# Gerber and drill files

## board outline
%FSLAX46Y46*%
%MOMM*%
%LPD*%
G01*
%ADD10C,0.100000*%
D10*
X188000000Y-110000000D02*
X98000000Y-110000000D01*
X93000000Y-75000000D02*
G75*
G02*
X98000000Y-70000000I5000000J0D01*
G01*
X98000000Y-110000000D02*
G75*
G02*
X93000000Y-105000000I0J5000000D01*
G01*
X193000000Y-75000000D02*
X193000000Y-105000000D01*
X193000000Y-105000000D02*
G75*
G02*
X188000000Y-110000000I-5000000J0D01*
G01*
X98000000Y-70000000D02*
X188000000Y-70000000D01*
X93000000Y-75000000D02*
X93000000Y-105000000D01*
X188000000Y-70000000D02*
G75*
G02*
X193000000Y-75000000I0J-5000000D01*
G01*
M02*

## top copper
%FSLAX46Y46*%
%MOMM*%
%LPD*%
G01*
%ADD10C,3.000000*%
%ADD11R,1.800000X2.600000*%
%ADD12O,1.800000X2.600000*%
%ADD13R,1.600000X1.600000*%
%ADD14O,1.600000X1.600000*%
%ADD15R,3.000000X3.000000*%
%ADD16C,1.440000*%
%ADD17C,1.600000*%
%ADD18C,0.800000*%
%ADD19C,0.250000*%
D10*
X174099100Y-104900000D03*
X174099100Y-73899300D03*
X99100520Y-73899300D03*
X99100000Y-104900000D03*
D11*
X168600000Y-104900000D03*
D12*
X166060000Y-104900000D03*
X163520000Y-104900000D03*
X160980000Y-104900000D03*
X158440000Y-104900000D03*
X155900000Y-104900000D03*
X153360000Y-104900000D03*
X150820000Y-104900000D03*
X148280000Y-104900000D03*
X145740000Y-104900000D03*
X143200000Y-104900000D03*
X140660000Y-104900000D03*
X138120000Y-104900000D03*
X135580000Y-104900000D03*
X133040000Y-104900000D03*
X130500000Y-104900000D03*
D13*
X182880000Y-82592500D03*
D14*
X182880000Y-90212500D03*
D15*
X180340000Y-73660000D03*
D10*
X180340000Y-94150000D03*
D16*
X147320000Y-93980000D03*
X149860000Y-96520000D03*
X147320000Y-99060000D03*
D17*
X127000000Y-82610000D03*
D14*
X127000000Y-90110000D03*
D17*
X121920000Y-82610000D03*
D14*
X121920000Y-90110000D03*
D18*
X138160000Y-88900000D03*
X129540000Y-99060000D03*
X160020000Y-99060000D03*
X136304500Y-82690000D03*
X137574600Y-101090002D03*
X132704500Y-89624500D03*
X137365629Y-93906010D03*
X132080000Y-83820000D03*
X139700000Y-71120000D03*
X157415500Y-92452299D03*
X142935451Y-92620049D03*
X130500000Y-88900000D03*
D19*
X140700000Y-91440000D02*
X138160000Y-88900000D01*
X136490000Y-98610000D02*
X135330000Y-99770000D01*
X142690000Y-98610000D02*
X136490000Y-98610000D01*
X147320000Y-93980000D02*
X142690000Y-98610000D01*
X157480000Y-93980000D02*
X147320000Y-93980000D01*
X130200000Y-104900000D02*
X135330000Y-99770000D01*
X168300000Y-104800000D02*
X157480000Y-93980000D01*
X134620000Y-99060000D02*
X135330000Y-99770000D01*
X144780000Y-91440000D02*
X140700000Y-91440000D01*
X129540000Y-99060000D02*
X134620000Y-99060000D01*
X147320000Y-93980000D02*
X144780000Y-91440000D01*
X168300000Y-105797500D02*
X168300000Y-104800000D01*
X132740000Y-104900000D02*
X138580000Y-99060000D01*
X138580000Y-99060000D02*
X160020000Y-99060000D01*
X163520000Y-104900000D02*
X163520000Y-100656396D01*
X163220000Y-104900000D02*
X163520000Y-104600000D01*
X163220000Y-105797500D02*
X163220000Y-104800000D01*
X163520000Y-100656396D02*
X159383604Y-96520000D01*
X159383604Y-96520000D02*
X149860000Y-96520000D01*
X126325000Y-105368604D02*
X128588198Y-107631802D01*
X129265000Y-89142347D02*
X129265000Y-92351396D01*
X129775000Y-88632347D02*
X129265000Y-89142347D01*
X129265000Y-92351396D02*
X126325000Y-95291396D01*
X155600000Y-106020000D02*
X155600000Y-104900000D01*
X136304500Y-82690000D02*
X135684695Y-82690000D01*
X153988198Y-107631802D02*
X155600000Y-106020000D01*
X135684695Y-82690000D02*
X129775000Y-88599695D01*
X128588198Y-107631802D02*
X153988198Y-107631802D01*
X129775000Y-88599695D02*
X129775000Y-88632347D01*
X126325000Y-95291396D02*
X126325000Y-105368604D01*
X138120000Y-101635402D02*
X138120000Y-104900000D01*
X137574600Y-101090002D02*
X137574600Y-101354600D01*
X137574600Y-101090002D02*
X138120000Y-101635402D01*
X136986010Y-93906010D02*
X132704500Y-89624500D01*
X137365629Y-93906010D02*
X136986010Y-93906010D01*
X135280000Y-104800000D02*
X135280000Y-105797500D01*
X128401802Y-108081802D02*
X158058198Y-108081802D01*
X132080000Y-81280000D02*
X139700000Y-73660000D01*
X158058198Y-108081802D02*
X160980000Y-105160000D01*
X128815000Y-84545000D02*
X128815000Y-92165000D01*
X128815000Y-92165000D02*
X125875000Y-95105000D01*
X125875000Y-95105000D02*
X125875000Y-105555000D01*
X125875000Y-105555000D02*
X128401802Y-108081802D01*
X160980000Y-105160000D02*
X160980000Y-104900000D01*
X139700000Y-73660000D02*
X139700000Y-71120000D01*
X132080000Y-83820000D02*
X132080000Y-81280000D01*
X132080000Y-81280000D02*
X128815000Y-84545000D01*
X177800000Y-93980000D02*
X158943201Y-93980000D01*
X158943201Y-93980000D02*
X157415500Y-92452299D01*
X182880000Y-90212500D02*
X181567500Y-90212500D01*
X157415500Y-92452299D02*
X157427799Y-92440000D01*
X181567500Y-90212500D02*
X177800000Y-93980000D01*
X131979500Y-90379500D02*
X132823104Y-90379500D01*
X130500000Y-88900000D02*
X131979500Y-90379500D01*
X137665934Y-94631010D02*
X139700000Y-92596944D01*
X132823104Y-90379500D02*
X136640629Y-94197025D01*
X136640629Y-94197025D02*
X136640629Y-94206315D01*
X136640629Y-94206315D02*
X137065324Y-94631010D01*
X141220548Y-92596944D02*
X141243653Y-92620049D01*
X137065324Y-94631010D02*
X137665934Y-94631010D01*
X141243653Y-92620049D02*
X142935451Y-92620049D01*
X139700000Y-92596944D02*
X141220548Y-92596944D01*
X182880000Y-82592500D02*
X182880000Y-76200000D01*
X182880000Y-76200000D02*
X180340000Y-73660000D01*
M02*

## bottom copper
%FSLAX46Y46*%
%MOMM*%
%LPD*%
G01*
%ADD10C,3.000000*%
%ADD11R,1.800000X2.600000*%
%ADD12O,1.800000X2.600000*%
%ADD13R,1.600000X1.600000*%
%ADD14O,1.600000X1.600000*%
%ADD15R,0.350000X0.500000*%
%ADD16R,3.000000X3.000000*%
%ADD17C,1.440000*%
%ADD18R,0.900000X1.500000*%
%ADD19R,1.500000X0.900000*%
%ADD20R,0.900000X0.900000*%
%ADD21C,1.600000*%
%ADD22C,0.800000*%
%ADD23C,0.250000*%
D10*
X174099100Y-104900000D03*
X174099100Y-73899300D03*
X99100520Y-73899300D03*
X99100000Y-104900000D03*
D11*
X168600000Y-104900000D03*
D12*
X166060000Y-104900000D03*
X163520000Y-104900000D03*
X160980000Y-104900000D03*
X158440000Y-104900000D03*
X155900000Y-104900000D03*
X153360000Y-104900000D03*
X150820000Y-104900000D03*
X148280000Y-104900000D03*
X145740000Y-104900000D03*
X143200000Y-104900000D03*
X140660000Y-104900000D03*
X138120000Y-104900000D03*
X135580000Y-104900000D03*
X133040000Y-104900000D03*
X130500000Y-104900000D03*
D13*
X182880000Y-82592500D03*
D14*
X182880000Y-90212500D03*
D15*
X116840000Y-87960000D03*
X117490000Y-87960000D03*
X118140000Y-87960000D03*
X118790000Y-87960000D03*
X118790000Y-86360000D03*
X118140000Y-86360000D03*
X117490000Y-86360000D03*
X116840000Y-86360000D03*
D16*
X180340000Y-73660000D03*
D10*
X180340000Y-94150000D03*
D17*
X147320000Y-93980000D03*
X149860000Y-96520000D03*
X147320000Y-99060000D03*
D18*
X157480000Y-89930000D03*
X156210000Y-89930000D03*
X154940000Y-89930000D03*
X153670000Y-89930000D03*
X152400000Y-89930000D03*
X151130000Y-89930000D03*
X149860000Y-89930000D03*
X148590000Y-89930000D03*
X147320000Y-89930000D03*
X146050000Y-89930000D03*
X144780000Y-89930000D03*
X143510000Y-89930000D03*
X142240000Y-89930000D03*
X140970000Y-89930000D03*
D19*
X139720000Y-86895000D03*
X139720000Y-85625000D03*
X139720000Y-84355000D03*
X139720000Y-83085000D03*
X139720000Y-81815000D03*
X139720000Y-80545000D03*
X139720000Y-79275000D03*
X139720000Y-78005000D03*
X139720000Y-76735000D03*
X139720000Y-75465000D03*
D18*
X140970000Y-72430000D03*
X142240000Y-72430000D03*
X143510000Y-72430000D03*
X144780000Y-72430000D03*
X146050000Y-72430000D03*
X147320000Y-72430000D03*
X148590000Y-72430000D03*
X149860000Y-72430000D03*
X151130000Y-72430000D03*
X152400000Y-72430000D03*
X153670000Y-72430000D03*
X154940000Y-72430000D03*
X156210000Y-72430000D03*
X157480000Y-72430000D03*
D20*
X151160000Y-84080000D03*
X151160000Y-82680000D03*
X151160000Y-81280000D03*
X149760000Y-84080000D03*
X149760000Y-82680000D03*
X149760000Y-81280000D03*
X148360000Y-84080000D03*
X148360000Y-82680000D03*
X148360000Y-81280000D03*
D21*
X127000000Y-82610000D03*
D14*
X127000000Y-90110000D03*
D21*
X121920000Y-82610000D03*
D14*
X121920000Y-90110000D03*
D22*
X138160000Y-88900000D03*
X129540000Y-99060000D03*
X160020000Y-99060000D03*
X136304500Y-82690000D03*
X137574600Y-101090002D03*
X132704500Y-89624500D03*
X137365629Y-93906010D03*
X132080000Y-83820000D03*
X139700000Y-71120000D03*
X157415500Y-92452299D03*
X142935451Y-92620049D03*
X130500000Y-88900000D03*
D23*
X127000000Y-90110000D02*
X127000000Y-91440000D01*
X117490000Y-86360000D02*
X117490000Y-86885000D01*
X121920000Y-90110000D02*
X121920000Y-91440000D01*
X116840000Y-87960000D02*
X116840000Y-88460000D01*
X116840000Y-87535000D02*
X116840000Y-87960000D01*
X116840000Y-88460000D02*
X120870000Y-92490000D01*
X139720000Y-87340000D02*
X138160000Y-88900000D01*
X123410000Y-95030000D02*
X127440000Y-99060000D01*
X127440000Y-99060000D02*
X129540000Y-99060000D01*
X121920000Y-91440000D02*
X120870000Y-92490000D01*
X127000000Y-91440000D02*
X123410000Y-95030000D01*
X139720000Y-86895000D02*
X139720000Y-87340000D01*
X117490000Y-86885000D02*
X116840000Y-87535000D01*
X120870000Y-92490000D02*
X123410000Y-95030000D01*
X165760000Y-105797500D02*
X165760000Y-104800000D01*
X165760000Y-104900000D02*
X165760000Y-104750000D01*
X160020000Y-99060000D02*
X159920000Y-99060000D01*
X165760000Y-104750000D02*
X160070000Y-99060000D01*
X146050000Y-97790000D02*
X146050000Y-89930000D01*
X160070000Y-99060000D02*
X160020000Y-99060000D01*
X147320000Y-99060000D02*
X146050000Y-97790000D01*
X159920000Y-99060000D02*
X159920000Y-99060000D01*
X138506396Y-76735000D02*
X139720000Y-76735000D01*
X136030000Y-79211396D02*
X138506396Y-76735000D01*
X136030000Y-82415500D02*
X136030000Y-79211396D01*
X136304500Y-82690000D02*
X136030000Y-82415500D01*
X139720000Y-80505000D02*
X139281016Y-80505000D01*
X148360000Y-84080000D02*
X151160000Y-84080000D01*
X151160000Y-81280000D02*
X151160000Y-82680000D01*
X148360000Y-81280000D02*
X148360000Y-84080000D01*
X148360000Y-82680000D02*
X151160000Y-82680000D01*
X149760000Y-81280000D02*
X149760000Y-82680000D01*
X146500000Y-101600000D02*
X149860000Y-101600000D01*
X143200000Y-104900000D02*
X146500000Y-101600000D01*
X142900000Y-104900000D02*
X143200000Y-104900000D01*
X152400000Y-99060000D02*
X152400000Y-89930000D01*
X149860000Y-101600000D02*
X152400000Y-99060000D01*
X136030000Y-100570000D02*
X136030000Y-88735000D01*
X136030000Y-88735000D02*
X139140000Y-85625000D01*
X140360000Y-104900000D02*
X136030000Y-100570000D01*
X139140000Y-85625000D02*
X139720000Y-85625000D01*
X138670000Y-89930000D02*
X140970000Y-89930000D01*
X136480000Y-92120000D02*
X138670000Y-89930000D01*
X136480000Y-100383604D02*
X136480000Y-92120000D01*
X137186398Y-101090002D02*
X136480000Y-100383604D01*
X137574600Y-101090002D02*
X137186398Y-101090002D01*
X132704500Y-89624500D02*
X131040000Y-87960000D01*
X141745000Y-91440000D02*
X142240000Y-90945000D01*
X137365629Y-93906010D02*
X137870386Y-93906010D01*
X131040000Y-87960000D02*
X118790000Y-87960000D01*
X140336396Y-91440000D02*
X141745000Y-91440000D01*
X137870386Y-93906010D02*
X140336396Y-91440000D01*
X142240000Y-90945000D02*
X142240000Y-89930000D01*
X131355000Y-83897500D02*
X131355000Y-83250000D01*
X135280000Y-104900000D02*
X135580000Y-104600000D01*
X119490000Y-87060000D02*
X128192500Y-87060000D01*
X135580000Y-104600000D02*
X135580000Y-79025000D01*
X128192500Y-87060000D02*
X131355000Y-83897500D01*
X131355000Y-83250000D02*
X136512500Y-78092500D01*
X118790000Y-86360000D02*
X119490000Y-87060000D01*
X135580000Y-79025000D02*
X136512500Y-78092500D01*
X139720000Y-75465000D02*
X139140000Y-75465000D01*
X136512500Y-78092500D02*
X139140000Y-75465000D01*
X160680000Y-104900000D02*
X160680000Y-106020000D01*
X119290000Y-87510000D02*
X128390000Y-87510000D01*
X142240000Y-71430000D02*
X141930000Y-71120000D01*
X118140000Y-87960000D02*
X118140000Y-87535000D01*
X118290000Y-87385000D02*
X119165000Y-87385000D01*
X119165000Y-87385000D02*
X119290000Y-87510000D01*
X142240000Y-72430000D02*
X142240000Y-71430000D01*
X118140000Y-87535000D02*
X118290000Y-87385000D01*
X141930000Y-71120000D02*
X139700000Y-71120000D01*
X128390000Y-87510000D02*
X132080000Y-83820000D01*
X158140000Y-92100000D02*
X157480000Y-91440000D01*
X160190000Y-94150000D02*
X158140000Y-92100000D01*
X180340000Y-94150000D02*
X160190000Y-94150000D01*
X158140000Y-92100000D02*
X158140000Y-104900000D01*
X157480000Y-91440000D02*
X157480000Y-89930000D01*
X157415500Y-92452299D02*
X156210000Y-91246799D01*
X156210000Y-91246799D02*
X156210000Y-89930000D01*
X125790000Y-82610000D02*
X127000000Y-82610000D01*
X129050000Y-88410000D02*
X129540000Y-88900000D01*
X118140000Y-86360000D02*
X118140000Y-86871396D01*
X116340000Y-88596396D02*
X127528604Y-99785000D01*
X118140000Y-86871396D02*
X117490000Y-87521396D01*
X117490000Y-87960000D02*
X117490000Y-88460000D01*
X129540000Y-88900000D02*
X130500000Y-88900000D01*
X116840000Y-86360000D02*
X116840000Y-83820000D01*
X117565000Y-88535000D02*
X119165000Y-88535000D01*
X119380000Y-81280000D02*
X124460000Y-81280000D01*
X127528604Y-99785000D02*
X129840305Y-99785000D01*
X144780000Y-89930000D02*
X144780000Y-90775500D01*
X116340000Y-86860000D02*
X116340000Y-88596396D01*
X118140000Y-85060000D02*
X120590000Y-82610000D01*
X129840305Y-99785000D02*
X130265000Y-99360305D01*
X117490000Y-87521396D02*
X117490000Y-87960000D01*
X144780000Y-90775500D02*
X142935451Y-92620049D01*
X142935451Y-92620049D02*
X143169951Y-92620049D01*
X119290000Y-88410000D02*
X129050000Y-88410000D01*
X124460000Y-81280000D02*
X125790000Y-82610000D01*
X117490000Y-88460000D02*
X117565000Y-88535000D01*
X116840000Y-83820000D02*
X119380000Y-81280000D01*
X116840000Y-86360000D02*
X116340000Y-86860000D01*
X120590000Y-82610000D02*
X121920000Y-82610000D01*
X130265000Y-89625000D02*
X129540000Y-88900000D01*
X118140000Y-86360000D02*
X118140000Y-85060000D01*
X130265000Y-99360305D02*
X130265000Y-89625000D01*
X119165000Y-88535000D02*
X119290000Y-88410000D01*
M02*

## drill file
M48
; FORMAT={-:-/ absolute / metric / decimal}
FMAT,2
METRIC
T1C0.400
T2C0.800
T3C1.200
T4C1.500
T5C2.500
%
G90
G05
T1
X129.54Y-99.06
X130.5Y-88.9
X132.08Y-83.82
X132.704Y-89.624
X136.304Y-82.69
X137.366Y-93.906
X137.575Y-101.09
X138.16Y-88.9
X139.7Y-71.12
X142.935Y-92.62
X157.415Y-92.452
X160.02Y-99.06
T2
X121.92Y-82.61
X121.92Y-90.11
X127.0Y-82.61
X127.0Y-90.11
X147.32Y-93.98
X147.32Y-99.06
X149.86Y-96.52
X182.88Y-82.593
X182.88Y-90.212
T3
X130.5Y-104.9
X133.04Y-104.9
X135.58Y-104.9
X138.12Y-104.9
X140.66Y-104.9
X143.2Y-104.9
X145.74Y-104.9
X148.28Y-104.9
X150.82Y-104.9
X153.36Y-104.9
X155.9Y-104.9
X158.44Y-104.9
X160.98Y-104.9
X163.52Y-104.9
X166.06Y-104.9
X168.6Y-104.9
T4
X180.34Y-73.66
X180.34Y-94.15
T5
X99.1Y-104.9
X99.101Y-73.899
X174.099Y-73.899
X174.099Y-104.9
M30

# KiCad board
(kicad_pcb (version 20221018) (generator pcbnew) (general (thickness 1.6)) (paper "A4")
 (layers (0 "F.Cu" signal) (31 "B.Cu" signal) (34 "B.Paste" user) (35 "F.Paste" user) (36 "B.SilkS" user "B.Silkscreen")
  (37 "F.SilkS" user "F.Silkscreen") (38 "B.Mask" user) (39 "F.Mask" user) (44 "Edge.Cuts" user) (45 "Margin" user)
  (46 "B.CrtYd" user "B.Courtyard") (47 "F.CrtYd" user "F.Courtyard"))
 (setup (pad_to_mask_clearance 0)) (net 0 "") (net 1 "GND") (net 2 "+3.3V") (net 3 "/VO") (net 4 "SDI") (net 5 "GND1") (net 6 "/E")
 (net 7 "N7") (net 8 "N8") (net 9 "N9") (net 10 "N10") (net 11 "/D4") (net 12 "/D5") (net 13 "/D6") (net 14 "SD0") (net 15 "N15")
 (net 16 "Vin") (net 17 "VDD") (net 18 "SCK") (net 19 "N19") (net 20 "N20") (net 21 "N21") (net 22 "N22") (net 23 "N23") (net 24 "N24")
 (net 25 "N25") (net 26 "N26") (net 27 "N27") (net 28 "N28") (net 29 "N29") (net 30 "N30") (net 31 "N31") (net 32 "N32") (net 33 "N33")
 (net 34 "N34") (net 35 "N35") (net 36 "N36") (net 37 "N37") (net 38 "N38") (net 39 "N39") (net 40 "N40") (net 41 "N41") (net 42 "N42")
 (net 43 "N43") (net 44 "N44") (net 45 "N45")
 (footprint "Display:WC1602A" (layer "F.Cu") (at 168.6 104.9 180)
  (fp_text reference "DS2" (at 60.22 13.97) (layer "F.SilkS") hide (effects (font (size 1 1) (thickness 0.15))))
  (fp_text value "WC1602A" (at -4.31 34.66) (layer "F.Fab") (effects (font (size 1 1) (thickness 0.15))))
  (pad "" thru_hole circle (at -5.4991 0 180) (size 3 3) (drill 2.5) (layers "*.Cu" "*.Mask"))
  (pad "" thru_hole circle (at -5.4991 31.0007 180) (size 3 3) (drill 2.5) (layers "*.Cu" "*.Mask"))
  (pad "" thru_hole circle (at 69.49948 31.0007 180) (size 3 3) (drill 2.5) (layers "*.Cu" "*.Mask"))
  (pad "" thru_hole circle (at 69.5 0 180) (size 3 3) (drill 2.5) (layers "*.Cu" "*.Mask"))
  (pad "1" thru_hole rect (at 0 0 180) (size 1.8 2.6) (drill 1.2) (layers "*.Cu" "*.Mask") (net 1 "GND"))
  (pad "2" thru_hole oval (at 2.54 0 180) (size 1.8 2.6) (drill 1.2) (layers "*.Cu" "*.Mask") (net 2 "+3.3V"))
  (pad "3" thru_hole oval (at 5.08 0 180) (size 1.8 2.6) (drill 1.2) (layers "*.Cu" "*.Mask") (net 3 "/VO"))
  (pad "4" thru_hole oval (at 7.62 0 180) (size 1.8 2.6) (drill 1.2) (layers "*.Cu" "*.Mask") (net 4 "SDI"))
  (pad "5" thru_hole oval (at 10.16 0 180) (size 1.8 2.6) (drill 1.2) (layers "*.Cu" "*.Mask") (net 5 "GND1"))
  (pad "6" thru_hole oval (at 12.7 0 180) (size 1.8 2.6) (drill 1.2) (layers "*.Cu" "*.Mask") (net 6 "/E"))
  (pad "7" thru_hole oval (at 15.24 0 180) (size 1.8 2.6) (drill 1.2) (layers "*.Cu" "*.Mask") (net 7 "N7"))
  (pad "8" thru_hole oval (at 17.78 0 180) (size 1.8 2.6) (drill 1.2) (layers "*.Cu" "*.Mask") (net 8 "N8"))
  (pad "9" thru_hole oval (at 20.32 0 180) (size 1.8 2.6) (drill 1.2) (layers "*.Cu" "*.Mask") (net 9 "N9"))
  (pad "10" thru_hole oval (at 22.86 0 180) (size 1.8 2.6) (drill 1.2) (layers "*.Cu" "*.Mask") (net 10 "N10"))
  (pad "11" thru_hole oval (at 25.4 0 180) (size 1.8 2.6) (drill 1.2) (layers "*.Cu" "*.Mask") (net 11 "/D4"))
  (pad "12" thru_hole oval (at 27.94 0 180) (size 1.8 2.6) (drill 1.2) (layers "*.Cu" "*.Mask") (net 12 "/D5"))
  (pad "13" thru_hole oval (at 30.48 0 180) (size 1.8 2.6) (drill 1.2) (layers "*.Cu" "*.Mask") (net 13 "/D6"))
  (pad "14" thru_hole oval (at 33.02 0 180) (size 1.8 2.6) (drill 1.2) (layers "*.Cu" "*.Mask") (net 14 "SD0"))
  (pad "15" thru_hole oval (at 35.56 0 180) (size 1.8 2.6) (drill 1.2) (layers "*.Cu" "*.Mask") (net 2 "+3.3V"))
  (pad "16" thru_hole oval (at 38.1 0 180) (size 1.8 2.6) (drill 1.2) (layers "*.Cu" "*.Mask") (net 1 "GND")))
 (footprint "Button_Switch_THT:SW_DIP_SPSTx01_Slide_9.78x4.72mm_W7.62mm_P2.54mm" (layer "F.Cu") (at 182.88 82.5925 -90)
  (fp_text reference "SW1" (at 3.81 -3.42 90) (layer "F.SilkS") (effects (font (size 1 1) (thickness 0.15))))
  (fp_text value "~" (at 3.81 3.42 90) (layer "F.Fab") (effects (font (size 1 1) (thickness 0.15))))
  (pad "1" thru_hole rect (at 0 0 270) (size 1.6 1.6) (drill 0.8) (layers "*.Cu" "*.Mask") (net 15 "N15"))
  (pad "2" thru_hole oval (at 7.62 0 270) (size 1.6 1.6) (drill 0.8) (layers "*.Cu" "*.Mask") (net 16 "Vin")))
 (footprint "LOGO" (layer "F.Cu") (at 185.42 101.6)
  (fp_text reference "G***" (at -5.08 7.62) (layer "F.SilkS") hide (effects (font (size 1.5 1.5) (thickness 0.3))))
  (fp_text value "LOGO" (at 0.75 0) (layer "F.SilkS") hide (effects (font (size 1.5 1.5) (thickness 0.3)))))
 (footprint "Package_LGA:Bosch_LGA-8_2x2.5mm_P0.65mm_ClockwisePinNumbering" (layer "B.Cu") (at 117.815 87.16)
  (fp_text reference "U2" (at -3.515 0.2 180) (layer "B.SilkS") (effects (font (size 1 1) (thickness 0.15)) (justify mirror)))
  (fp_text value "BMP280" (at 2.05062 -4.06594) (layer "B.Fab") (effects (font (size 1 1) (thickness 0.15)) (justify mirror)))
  (pad "1" smd rect (at -0.975 0.8 270) (size 0.5 0.35) (layers "B.Cu" "B.Paste" "B.Mask") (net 1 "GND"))
  (pad "2" smd rect (at -0.325 0.8 270) (size 0.5 0.35) (layers "B.Cu" "B.Paste" "B.Mask") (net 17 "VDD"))
  (pad "3" smd rect (at 0.325 0.8 270) (size 0.5 0.35) (layers "B.Cu" "B.Paste" "B.Mask") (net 4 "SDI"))
  (pad "4" smd rect (at 0.975 0.8 270) (size 0.5 0.35) (layers "B.Cu" "B.Paste" "B.Mask") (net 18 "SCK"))
  (pad "5" smd rect (at 0.975 -0.8 270) (size 0.5 0.35) (layers "B.Cu" "B.Paste" "B.Mask") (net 14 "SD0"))
  (pad "6" smd rect (at 0.325 -0.8 270) (size 0.5 0.35) (layers "B.Cu" "B.Paste" "B.Mask") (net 17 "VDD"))
  (pad "7" smd rect (at -0.325 -0.8 270) (size 0.5 0.35) (layers "B.Cu" "B.Paste" "B.Mask") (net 1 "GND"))
  (pad "8" smd rect (at -0.975 -0.8 270) (size 0.5 0.35) (layers "B.Cu" "B.Paste" "B.Mask") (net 17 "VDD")))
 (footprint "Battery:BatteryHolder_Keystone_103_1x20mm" (layer "B.Cu") (at 180.34 73.66 -90)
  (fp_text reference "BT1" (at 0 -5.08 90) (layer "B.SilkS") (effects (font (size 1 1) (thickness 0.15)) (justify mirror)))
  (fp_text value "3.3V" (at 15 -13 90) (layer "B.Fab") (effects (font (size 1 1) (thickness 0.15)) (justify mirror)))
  (pad "1" thru_hole rect (at 0 0 270) (size 3 3) (drill 1.5) (layers "*.Cu" "*.Mask") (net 15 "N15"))
  (pad "2" thru_hole circle (at 20.49 0 270) (size 3 3) (drill 1.5) (layers "*.Cu" "*.Mask") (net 5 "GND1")))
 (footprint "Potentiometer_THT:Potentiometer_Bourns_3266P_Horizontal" (layer "B.Cu") (at 147.32 93.98 180)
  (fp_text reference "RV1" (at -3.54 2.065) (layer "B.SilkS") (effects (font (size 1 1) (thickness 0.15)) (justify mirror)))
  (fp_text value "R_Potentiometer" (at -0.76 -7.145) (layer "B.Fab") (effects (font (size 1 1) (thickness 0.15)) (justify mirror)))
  (pad "1" thru_hole circle (at 0 0 180) (size 1.44 1.44) (drill 0.8) (layers "*.Cu" "*.Mask") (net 1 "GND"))
  (pad "2" thru_hole circle (at -2.54 -2.54 180) (size 1.44 1.44) (drill 0.8) (layers "*.Cu" "*.Mask") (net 3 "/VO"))
  (pad "3" thru_hole circle (at 0 -5.08 180) (size 1.44 1.44) (drill 0.8) (layers "*.Cu" "*.Mask") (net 2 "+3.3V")))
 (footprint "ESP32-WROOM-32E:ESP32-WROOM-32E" (layer "B.Cu") (at 149.225 81.18 90)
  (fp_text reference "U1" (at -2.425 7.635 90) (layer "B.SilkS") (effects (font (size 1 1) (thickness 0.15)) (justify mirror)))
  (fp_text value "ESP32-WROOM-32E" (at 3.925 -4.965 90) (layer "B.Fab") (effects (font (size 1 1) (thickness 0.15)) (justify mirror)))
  (pad "1" smd rect (at -8.75 8.255 90) (size 1.5 0.9) (layers "B.Cu" "B.Paste" "B.Mask") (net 5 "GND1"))
  (pad "2" smd rect (at -8.75 6.985 90) (size 1.5 0.9) (layers "B.Cu" "B.Paste" "B.Mask") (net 16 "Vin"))
  (pad "3" smd rect (at -8.75 5.715 90) (size 1.5 0.9) (layers "B.Cu" "B.Paste" "B.Mask") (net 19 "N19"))
  (pad "4" smd rect (at -8.75 4.445 90) (size 1.5 0.9) (layers "B.Cu" "B.Paste" "B.Mask") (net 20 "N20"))
  (pad "5" smd rect (at -8.75 3.175 90) (size 1.5 0.9) (layers "B.Cu" "B.Paste" "B.Mask") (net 11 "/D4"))
  (pad "6" smd rect (at -8.75 1.905 90) (size 1.5 0.9) (layers "B.Cu" "B.Paste" "B.Mask") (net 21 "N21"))
  (pad "7" smd rect (at -8.75 0.635 90) (size 1.5 0.9) (layers "B.Cu" "B.Paste" "B.Mask") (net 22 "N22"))
  (pad "8" smd rect (at -8.75 -0.635 90) (size 1.5 0.9) (layers "B.Cu" "B.Paste" "B.Mask") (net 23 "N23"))
  (pad "9" smd rect (at -8.75 -1.905 90) (size 1.5 0.9) (layers "B.Cu" "B.Paste" "B.Mask") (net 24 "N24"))
  (pad "10" smd rect (at -8.75 -3.175 90) (size 1.5 0.9) (layers "B.Cu" "B.Paste" "B.Mask") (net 2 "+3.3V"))
  (pad "11" smd rect (at -8.75 -4.445 90) (size 1.5 0.9) (layers "B.Cu" "B.Paste" "B.Mask") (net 17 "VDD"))
  (pad "12" smd rect (at -8.75 -5.715 90) (size 1.5 0.9) (layers "B.Cu" "B.Paste" "B.Mask") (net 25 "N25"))
  (pad "13" smd rect (at -8.75 -6.985 90) (size 1.5 0.9) (layers "B.Cu" "B.Paste" "B.Mask") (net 18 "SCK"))
  (pad "14" smd rect (at -8.75 -8.255 90) (size 1.5 0.9) (layers "B.Cu" "B.Paste" "B.Mask") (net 13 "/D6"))
  (pad "15" smd rect (at -5.715 -9.505) (size 1.5 0.9) (layers "B.Cu" "B.Paste" "B.Mask") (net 1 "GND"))
  (pad "16" smd rect (at -4.445 -9.505) (size 1.5 0.9) (layers "B.Cu" "B.Paste" "B.Mask") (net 12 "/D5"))
  (pad "17" smd rect (at -3.175 -9.505) (size 1.5 0.9) (layers "B.Cu" "B.Paste" "B.Mask") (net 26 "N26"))
  (pad "18" smd rect (at -1.905 -9.505) (size 1.5 0.9) (layers "B.Cu" "B.Paste" "B.Mask") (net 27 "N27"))
  (pad "19" smd rect (at -0.635 -9.505) (size 1.5 0.9) (layers "B.Cu" "B.Paste" "B.Mask") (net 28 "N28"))
  (pad "20" smd rect (at 0.635 -9.505) (size 1.5 0.9) (layers "B.Cu" "B.Paste" "B.Mask") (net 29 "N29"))
  (pad "21" smd rect (at 1.905 -9.505) (size 1.5 0.9) (layers "B.Cu" "B.Paste" "B.Mask") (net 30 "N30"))
  (pad "22" smd rect (at 3.175 -9.505) (size 1.5 0.9) (layers "B.Cu" "B.Paste" "B.Mask") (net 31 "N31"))
  (pad "23" smd rect (at 4.445 -9.505) (size 1.5 0.9) (layers "B.Cu" "B.Paste" "B.Mask") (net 6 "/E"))
  (pad "24" smd rect (at 5.715 -9.505) (size 1.5 0.9) (layers "B.Cu" "B.Paste" "B.Mask") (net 14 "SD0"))
  (pad "25" smd rect (at 8.75 -8.255 270) (size 1.5 0.9) (layers "B.Cu" "B.Paste" "B.Mask") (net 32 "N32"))
  (pad "26" smd rect (at 8.75 -6.985 270) (size 1.5 0.9) (layers "B.Cu" "B.Paste" "B.Mask") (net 4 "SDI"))
  (pad "27" smd rect (at 8.75 -5.715 270) (size 1.5 0.9) (layers "B.Cu" "B.Paste" "B.Mask") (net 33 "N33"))
  (pad "28" smd rect (at 8.75 -4.445 270) (size 1.5 0.9) (layers "B.Cu" "B.Paste" "B.Mask") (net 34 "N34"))
  (pad "29" smd rect (at 8.75 -3.175 270) (size 1.5 0.9) (layers "B.Cu" "B.Paste" "B.Mask") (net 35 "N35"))
  (pad "30" smd rect (at 8.75 -1.905 270) (size 1.5 0.9) (layers "B.Cu" "B.Paste" "B.Mask") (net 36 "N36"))
  (pad "31" smd rect (at 8.75 -0.635 270) (size 1.5 0.9) (layers "B.Cu" "B.Paste" "B.Mask") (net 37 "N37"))
  (pad "32" smd rect (at 8.75 0.635 270) (size 1.5 0.9) (layers "B.Cu" "B.Paste" "B.Mask") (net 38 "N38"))
  (pad "33" smd rect (at 8.75 1.905 270) (size 1.5 0.9) (layers "B.Cu" "B.Paste" "B.Mask") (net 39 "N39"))
  (pad "34" smd rect (at 8.75 3.175 270) (size 1.5 0.9) (layers "B.Cu" "B.Paste" "B.Mask") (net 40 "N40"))
  (pad "35" smd rect (at 8.75 4.445 270) (size 1.5 0.9) (layers "B.Cu" "B.Paste" "B.Mask") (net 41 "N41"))
  (pad "36" smd rect (at 8.75 5.715 270) (size 1.5 0.9) (layers "B.Cu" "B.Paste" "B.Mask") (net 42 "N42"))
  (pad "37" smd rect (at 8.75 6.985 270) (size 1.5 0.9) (layers "B.Cu" "B.Paste" "B.Mask") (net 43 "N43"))
  (pad "38" smd rect (at 8.75 8.255 270) (size 1.5 0.9) (layers "B.Cu" "B.Paste" "B.Mask") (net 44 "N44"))
  (pad "GND@39" smd rect (at -2.9 1.935 90) (size 0.9 0.9) (layers "B.Cu" "B.Paste" "B.Mask") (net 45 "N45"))
  (pad "GND@40" smd rect (at -1.5 1.935 90) (size 0.9 0.9) (layers "B.Cu" "B.Paste" "B.Mask") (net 45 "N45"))
  (pad "GND@41" smd rect (at -0.1 1.935 90) (size 0.9 0.9) (layers "B.Cu" "B.Paste" "B.Mask") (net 45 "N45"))
  (pad "GND@42" smd rect (at -2.9 0.535 90) (size 0.9 0.9) (layers "B.Cu" "B.Paste" "B.Mask") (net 45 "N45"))
  (pad "GND@43" smd rect (at -1.5 0.535 90) (size 0.9 0.9) (layers "B.Cu" "B.Paste" "B.Mask") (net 45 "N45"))
  (pad "GND@44" smd rect (at -0.1 0.535 90) (size 0.9 0.9) (layers "B.Cu" "B.Paste" "B.Mask") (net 45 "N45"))
  (pad "GND@45" smd rect (at -2.9 -0.865 90) (size 0.9 0.9) (layers "B.Cu" "B.Paste" "B.Mask") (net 45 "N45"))
  (pad "GND@46" smd rect (at -1.5 -0.865 90) (size 0.9 0.9) (layers "B.Cu" "B.Paste" "B.Mask") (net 45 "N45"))
  (pad "GND@47" smd rect (at -0.1 -0.865 90) (size 0.9 0.9) (layers "B.Cu" "B.Paste" "B.Mask") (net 45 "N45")))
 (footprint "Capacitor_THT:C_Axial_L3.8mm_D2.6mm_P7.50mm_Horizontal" (layer "B.Cu") (at 127 82.61 -90)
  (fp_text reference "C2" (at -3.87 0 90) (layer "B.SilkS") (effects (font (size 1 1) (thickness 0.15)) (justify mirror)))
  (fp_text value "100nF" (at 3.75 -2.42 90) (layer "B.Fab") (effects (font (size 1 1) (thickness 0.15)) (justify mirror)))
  (pad "1" thru_hole circle (at 0 0 270) (size 1.6 1.6) (drill 0.8) (layers "*.Cu" "*.Mask") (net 17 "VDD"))
  (pad "2" thru_hole oval (at 7.5 0 270) (size 1.6 1.6) (drill 0.8) (layers "*.Cu" "*.Mask") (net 1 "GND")))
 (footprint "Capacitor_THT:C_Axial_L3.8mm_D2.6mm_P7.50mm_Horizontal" (layer "B.Cu") (at 121.92 82.61 -90)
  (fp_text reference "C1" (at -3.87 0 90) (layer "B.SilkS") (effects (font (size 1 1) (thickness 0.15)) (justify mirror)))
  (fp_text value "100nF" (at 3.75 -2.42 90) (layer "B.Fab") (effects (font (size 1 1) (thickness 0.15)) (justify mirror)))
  (pad "1" thru_hole circle (at 0 0 270) (size 1.6 1.6) (drill 0.8) (layers "*.Cu" "*.Mask") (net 17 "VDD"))
  (pad "2" thru_hole oval (at 7.5 0 270) (size 1.6 1.6) (drill 0.8) (layers "*.Cu" "*.Mask") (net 1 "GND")))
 (gr_line (start 188 110) (end 98 110) (stroke (width 0.1) (type default)) (layer "Edge.Cuts"))
 (gr_arc (start 93 75) (mid 94.464466 71.464467) (end 98 70) (stroke (width 0.1) (type default)) (layer "Edge.Cuts"))
 (gr_arc (start 98 110) (mid 94.464467 108.535534) (end 93 105) (stroke (width 0.1) (type default)) (layer "Edge.Cuts"))
 (gr_line (start 193 75) (end 193 105) (stroke (width 0.1) (type default)) (layer "Edge.Cuts"))
 (gr_arc (start 193 105) (mid 191.535534 108.535533) (end 188 110) (stroke (width 0.1) (type default)) (layer "Edge.Cuts"))
 (gr_line (start 98 70) (end 188 70) (stroke (width 0.1) (type default)) (layer "Edge.Cuts"))
 (gr_line (start 93 75) (end 93 105) (stroke (width 0.1) (type default)) (layer "Edge.Cuts"))
 (gr_arc (start 188 70) (mid 191.535534 71.464466) (end 193 75) (stroke (width 0.1) (type default)) (layer "Edge.Cuts"))
 (segment (start 140.7 91.44) (end 138.16 88.9) (width 0.25) (layer "F.Cu") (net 1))
 (segment (start 136.49 98.61) (end 135.33 99.77) (width 0.25) (layer "F.Cu") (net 1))
 (segment (start 142.69 98.61) (end 136.49 98.61) (width 0.25) (layer "F.Cu") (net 1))
 (segment (start 147.32 93.98) (end 142.69 98.61) (width 0.25) (layer "F.Cu") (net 1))
 (segment (start 157.48 93.98) (end 147.32 93.98) (width 0.25) (layer "F.Cu") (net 1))
 (segment (start 130.2 104.9) (end 135.33 99.77) (width 0.25) (layer "F.Cu") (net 1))
 (segment (start 168.3 104.8) (end 157.48 93.98) (width 0.25) (layer "F.Cu") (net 1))
 (segment (start 134.62 99.06) (end 135.33 99.77) (width 0.25) (layer "F.Cu") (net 1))
 (segment (start 144.78 91.44) (end 140.7 91.44) (width 0.25) (layer "F.Cu") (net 1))
 (segment (start 129.54 99.06) (end 134.62 99.06) (width 0.25) (layer "F.Cu") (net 1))
 (segment (start 147.32 93.98) (end 144.78 91.44) (width 0.25) (layer "F.Cu") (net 1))
 (segment (start 168.3 105.7975) (end 168.3 104.8) (width 0.25) (layer "F.Cu") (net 1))
 (via (at 138.16 88.9) (size 0.8) (drill 0.4) (layers "F.Cu" "B.Cu") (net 1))
 (via (at 129.54 99.06) (size 0.8) (drill 0.4) (layers "F.Cu" "B.Cu") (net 1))
 (segment (start 127 90.11) (end 127 91.44) (width 0.25) (layer "B.Cu") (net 1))
 (segment (start 117.49 86.36) (end 117.49 86.885) (width 0.25) (layer "B.Cu") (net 1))
 (segment (start 121.92 90.11) (end 121.92 91.44) (width 0.25) (layer "B.Cu") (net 1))
 (segment (start 116.84 87.96) (end 116.84 88.46) (width 0.25) (layer "B.Cu") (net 1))
 (segment (start 116.84 87.535) (end 116.84 87.96) (width 0.25) (layer "B.Cu") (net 1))
 (segment (start 116.84 88.46) (end 120.87 92.49) (width 0.25) (layer "B.Cu") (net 1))
 (segment (start 139.72 87.34) (end 138.16 88.9) (width 0.25) (layer "B.Cu") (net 1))
 (segment (start 123.41 95.03) (end 127.44 99.06) (width 0.25) (layer "B.Cu") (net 1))
 (segment (start 127.44 99.06) (end 129.54 99.06) (width 0.25) (layer "B.Cu") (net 1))
 (segment (start 121.92 91.44) (end 120.87 92.49) (width 0.25) (layer "B.Cu") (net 1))
 (segment (start 127 91.44) (end 123.41 95.03) (width 0.25) (layer "B.Cu") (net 1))
 (segment (start 139.72 86.895) (end 139.72 87.34) (width 0.25) (layer "B.Cu") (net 1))
 (segment (start 117.49 86.885) (end 116.84 87.535) (width 0.25) (layer "B.Cu") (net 1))
 (segment (start 120.87 92.49) (end 123.41 95.03) (width 0.25) (layer "B.Cu") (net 1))
 (segment (start 132.74 104.9) (end 138.58 99.06) (width 0.25) (layer "F.Cu") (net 2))
 (segment (start 138.58 99.06) (end 160.02 99.06) (width 0.25) (layer "F.Cu") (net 2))
 (via (at 160.02 99.06) (size 0.8) (drill 0.4) (layers "F.Cu" "B.Cu") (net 2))
 (segment (start 165.76 105.7975) (end 165.76 104.8) (width 0.25) (layer "B.Cu") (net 2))
 (segment (start 165.76 104.9) (end 165.76 104.75) (width 0.25) (layer "B.Cu") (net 2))
 (segment (start 160.02 99.06) (end 159.92 99.06) (width 0.25) (layer "B.Cu") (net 2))
 (segment (start 165.76 104.75) (end 160.07 99.06) (width 0.25) (layer "B.Cu") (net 2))
 (segment (start 146.05 97.79) (end 146.05 89.93) (width 0.25) (layer "B.Cu") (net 2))
 (segment (start 160.07 99.06) (end 160.02 99.06) (width 0.25) (layer "B.Cu") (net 2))
 (segment (start 147.32 99.06) (end 146.05 97.79) (width 0.25) (layer "B.Cu") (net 2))
 (segment (start 159.92 99.06) (end 159.92 99.06) (width 0.25) (layer "B.Cu") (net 2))
 (segment (start 163.52 104.9) (end 163.52 100.656396) (width 0.25) (layer "F.Cu") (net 3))
 (segment (start 163.22 104.9) (end 163.52 104.6) (width 0.25) (layer "F.Cu") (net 3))
 (segment (start 163.22 105.7975) (end 163.22 104.8) (width 0.25) (layer "F.Cu") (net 3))
 (segment (start 163.52 100.656396) (end 159.383604 96.52) (width 0.25) (layer "F.Cu") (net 3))
 (segment (start 159.383604 96.52) (end 149.86 96.52) (width 0.25) (layer "F.Cu") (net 3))
 (segment (start 126.325 105.368604) (end 128.588198 107.631802) (width 0.25) (layer "F.Cu") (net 6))
 (segment (start 129.265 89.142347) (end 129.265 92.351396) (width 0.25) (layer "F.Cu") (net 6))
 (segment (start 129.775 88.632347) (end 129.265 89.142347) (width 0.25) (layer "F.Cu") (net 6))
 (segment (start 129.265 92.351396) (end 126.325 95.291396) (width 0.25) (layer "F.Cu") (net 6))
 (segment (start 155.6 106.02) (end 155.6 104.9) (width 0.25) (layer "F.Cu") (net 6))
 (segment (start 136.3045 82.69) (end 135.684695 82.69) (width 0.25) (layer "F.Cu") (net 6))
 (segment (start 153.988198 107.631802) (end 155.6 106.02) (width 0.25) (layer "F.Cu") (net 6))
 (segment (start 135.684695 82.69) (end 129.775 88.599695) (width 0.25) (layer "F.Cu") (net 6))
 (segment (start 128.588198 107.631802) (end 153.988198 107.631802) (width 0.25) (layer "F.Cu") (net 6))
 (segment (start 129.775 88.599695) (end 129.775 88.632347) (width 0.25) (layer "F.Cu") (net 6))
 (segment (start 126.325 95.291396) (end 126.325 105.368604) (width 0.25) (layer "F.Cu") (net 6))
 (via (at 136.3045 82.69) (size 0.8) (drill 0.4) (layers "F.Cu" "B.Cu") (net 6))
 (segment (start 138.506396 76.735) (end 139.72 76.735) (width 0.25) (layer "B.Cu") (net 6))
 (segment (start 136.03 79.211396) (end 138.506396 76.735) (width 0.25) (layer "B.Cu") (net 6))
 (segment (start 136.03 82.4155) (end 136.03 79.211396) (width 0.25) (layer "B.Cu") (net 6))
 (segment (start 136.3045 82.69) (end 136.03 82.4155) (width 0.25) (layer "B.Cu") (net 6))
 (segment (start 139.72 80.505) (end 139.281016 80.505) (width 0.25) (layer "B.Cu") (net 29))
 (segment (start 148.36 84.08) (end 151.16 84.08) (width 0.25) (layer "B.Cu") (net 45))
 (segment (start 151.16 81.28) (end 151.16 82.68) (width 0.25) (layer "B.Cu") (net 45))
 (segment (start 148.36 81.28) (end 148.36 84.08) (width 0.25) (layer "B.Cu") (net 45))
 (segment (start 148.36 82.68) (end 151.16 82.68) (width 0.25) (layer "B.Cu") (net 45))
 (segment (start 149.76 81.28) (end 149.76 82.68) (width 0.25) (layer "B.Cu") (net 45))
 (segment (start 146.5 101.6) (end 149.86 101.6) (width 0.25) (layer "B.Cu") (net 11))
 (segment (start 143.2 104.9) (end 146.5 101.6) (width 0.25) (layer "B.Cu") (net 11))
 (segment (start 142.9 104.9) (end 143.2 104.9) (width 0.25) (layer "B.Cu") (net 11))
 (segment (start 152.4 99.06) (end 152.4 89.93) (width 0.25) (layer "B.Cu") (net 11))
 (segment (start 149.86 101.6) (end 152.4 99.06) (width 0.25) (layer "B.Cu") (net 11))
 (segment (start 136.03 100.57) (end 136.03 88.735) (width 0.25) (layer "B.Cu") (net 12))
 (segment (start 136.03 88.735) (end 139.14 85.625) (width 0.25) (layer "B.Cu") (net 12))
 (segment (start 140.36 104.9) (end 136.03 100.57) (width 0.25) (layer "B.Cu") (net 12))
 (segment (start 139.14 85.625) (end 139.72 85.625) (width 0.25) (layer "B.Cu") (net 12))
 (segment (start 138.12 101.635402) (end 138.12 104.9) (width 0.25) (layer "F.Cu") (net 13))
 (segment (start 137.5746 101.090002) (end 137.5746 101.3546) (width 0.25) (layer "F.Cu") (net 13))
 (segment (start 137.5746 101.090002) (end 138.12 101.635402) (width 0.25) (layer "F.Cu") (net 13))
 (via (at 137.5746 101.090002) (size 0.8) (drill 0.4) (layers "F.Cu" "B.Cu") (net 13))
 (segment (start 138.67 89.93) (end 140.97 89.93) (width 0.25) (layer "B.Cu") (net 13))
 (segment (start 136.48 92.12) (end 138.67 89.93) (width 0.25) (layer "B.Cu") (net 13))
 (segment (start 136.48 100.383604) (end 136.48 92.12) (width 0.25) (layer "B.Cu") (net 13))
 (segment (start 137.186398 101.090002) (end 136.48 100.383604) (width 0.25) (layer "B.Cu") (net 13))
 (segment (start 137.5746 101.090002) (end 137.186398 101.090002) (width 0.25) (layer "B.Cu") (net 13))
 (segment (start 136.98601 93.90601) (end 132.7045 89.6245) (width 0.25) (layer "F.Cu") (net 18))
 (segment (start 137.365629 93.90601) (end 136.98601 93.90601) (width 0.25) (layer "F.Cu") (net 18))
 (via (at 132.7045 89.6245) (size 0.8) (drill 0.4) (layers "F.Cu" "B.Cu") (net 18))
 (via (at 137.365629 93.90601) (size 0.8) (drill 0.4) (layers "F.Cu" "B.Cu") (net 18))
 (segment (start 132.7045 89.6245) (end 131.04 87.96) (width 0.25) (layer "B.Cu") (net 18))
 (segment (start 141.745 91.44) (end 142.24 90.945) (width 0.25) (layer "B.Cu") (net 18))
 (segment (start 137.365629 93.90601) (end 137.870386 93.90601) (width 0.25) (layer "B.Cu") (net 18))
 (segment (start 131.04 87.96) (end 118.79 87.96) (width 0.25) (layer "B.Cu") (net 18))
 (segment (start 140.336396 91.44) (end 141.745 91.44) (width 0.25) (layer "B.Cu") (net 18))
 (segment (start 137.870386 93.90601) (end 140.336396 91.44) (width 0.25) (layer "B.Cu") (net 18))
 (segment (start 142.24 90.945) (end 142.24 89.93) (width 0.25) (layer "B.Cu") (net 18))
 (segment (start 135.28 104.8) (end 135.28 105.7975) (width 0.25) (layer "F.Cu") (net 14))
 (segment (start 131.355 83.8975) (end 131.355 83.25) (width 0.25) (layer "B.Cu") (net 14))
 (segment (start 135.28 104.9) (end 135.58 104.6) (width 0.25) (layer "B.Cu") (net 14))
 (segment (start 119.49 87.06) (end 128.1925 87.06) (width 0.25) (layer "B.Cu") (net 14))
 (segment (start 135.58 104.6) (end 135.58 79.025) (width 0.25) (layer "B.Cu") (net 14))
 (segment (start 128.1925 87.06) (end 131.355 83.8975) (width 0.25) (layer "B.Cu") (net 14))
 (segment (start 131.355 83.25) (end 136.5125 78.0925) (width 0.25) (layer "B.Cu") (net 14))
 (segment (start 118.79 86.36) (end 119.49 87.06) (width 0.25) (layer "B.Cu") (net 14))
 (segment (start 135.58 79.025) (end 136.5125 78.0925) (width 0.25) (layer "B.Cu") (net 14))
 (segment (start 139.72 75.465) (end 139.14 75.465) (width 0.25) (layer "B.Cu") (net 14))
 (segment (start 136.5125 78.0925) (end 139.14 75.465) (width 0.25) (layer "B.Cu") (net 14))
 (segment (start 128.401802 108.081802) (end 158.058198 108.081802) (width 0.25) (layer "F.Cu") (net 4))
 (segment (start 132.08 81.28) (end 139.7 73.66) (width 0.25) (layer "F.Cu") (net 4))
 (segment (start 158.058198 108.081802) (end 160.98 105.16) (width 0.25) (layer "F.Cu") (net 4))
 (segment (start 128.815 84.545) (end 128.815 92.165) (width 0.25) (layer "F.Cu") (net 4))
 (segment (start 128.815 92.165) (end 125.875 95.105) (width 0.25) (layer "F.Cu") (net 4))
 (segment (start 125.875 95.105) (end 125.875 105.555) (width 0.25) (layer "F.Cu") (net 4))
 (segment (start 125.875 105.555) (end 128.401802 108.081802) (width 0.25) (layer "F.Cu") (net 4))
 (segment (start 160.98 105.16) (end 160.98 104.9) (width 0.25) (layer "F.Cu") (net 4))
 (segment (start 139.7 73.66) (end 139.7 71.12) (width 0.25) (layer "F.Cu") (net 4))
 (segment (start 132.08 83.82) (end 132.08 81.28) (width 0.25) (layer "F.Cu") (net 4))
 (segment (start 132.08 81.28) (end 128.815 84.545) (width 0.25) (layer "F.Cu") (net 4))
 (via (at 132.08 83.82) (size 0.8) (drill 0.4) (layers "F.Cu" "B.Cu") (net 4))
 (via (at 139.7 71.12) (size 0.8) (drill 0.4) (layers "F.Cu" "B.Cu") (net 4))
 (segment (start 160.68 104.9) (end 160.68 106.02) (width 0.25) (layer "B.Cu") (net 4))
 (segment (start 119.29 87.51) (end 128.39 87.51) (width 0.25) (layer "B.Cu") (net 4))
 (segment (start 142.24 71.43) (end 141.93 71.12) (width 0.25) (layer "B.Cu") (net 4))
 (segment (start 118.14 87.96) (end 118.14 87.535) (width 0.25) (layer "B.Cu") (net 4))
 (segment (start 118.29 87.385) (end 119.165 87.385) (width 0.25) (layer "B.Cu") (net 4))
 (segment (start 119.165 87.385) (end 119.29 87.51) (width 0.25) (layer "B.Cu") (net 4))
 (segment (start 142.24 72.43) (end 142.24 71.43) (width 0.25) (layer "B.Cu") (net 4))
 (segment (start 118.14 87.535) (end 118.29 87.385) (width 0.25) (layer "B.Cu") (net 4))
 (segment (start 141.93 71.12) (end 139.7 71.12) (width 0.25) (layer "B.Cu") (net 4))
 (segment (start 128.39 87.51) (end 132.08 83.82) (width 0.25) (layer "B.Cu") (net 4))
 (segment (start 158.14 92.1) (end 157.48 91.44) (width 0.25) (layer "B.Cu") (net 5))
 (segment (start 160.19 94.15) (end 158.14 92.1) (width 0.25) (layer "B.Cu") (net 5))
 (segment (start 180.34 94.15) (end 160.19 94.15) (width 0.25) (layer "B.Cu") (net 5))
 (segment (start 158.14 92.1) (end 158.14 104.9) (width 0.25) (layer "B.Cu") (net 5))
 (segment (start 157.48 91.44) (end 157.48 89.93) (width 0.25) (layer "B.Cu") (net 5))
 (segment (start 177.8 93.98) (end 158.943201 93.98) (width 0.25) (layer "F.Cu") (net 16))
 (segment (start 158.943201 93.98) (end 157.4155 92.452299) (width 0.25) (layer "F.Cu") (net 16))
 (segment (start 182.88 90.2125) (end 181.5675 90.2125) (width 0.25) (layer "F.Cu") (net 16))
 (segment (start 157.4155 92.452299) (end 157.427799 92.44) (width 0.25) (layer "F.Cu") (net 16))
 (segment (start 181.5675 90.2125) (end 177.8 93.98) (width 0.25) (layer "F.Cu") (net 16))
 (via (at 157.4155 92.452299) (size 0.8) (drill 0.4) (layers "F.Cu" "B.Cu") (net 16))
 (segment (start 157.4155 92.452299) (end 156.21 91.246799) (width 0.25) (layer "B.Cu") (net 16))
 (segment (start 156.21 91.246799) (end 156.21 89.93) (width 0.25) (layer "B.Cu") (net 16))
 (segment (start 131.9795 90.3795) (end 132.823104 90.3795) (width 0.25) (layer "F.Cu") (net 17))
 (segment (start 130.5 88.9) (end 131.9795 90.3795) (width 0.25) (layer "F.Cu") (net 17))
 (segment (start 137.665934 94.63101) (end 139.7 92.596944) (width 0.25) (layer "F.Cu") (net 17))
 (segment (start 132.823104 90.3795) (end 136.640629 94.197025) (width 0.25) (layer "F.Cu") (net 17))
 (segment (start 136.640629 94.197025) (end 136.640629 94.206315) (width 0.25) (layer "F.Cu") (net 17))
 (segment (start 136.640629 94.206315) (end 137.065324 94.63101) (width 0.25) (layer "F.Cu") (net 17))
 (segment (start 141.220548 92.596944) (end 141.243653 92.620049) (width 0.25) (layer "F.Cu") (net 17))
 (segment (start 137.065324 94.63101) (end 137.665934 94.63101) (width 0.25) (layer "F.Cu") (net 17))
 (segment (start 141.243653 92.620049) (end 142.935451 92.620049) (width 0.25) (layer "F.Cu") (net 17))
 (segment (start 139.7 92.596944) (end 141.220548 92.596944) (width 0.25) (layer "F.Cu") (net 17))
 (via (at 142.935451 92.620049) (size 0.8) (drill 0.4) (layers "F.Cu" "B.Cu") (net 17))
 (via (at 130.5 88.9) (size 0.8) (drill 0.4) (layers "F.Cu" "B.Cu") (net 17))
 (segment (start 125.79 82.61) (end 127 82.61) (width 0.25) (layer "B.Cu") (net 17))
 (segment (start 129.05 88.41) (end 129.54 88.9) (width 0.25) (layer "B.Cu") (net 17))
 (segment (start 118.14 86.36) (end 118.14 86.871396) (width 0.25) (layer "B.Cu") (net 17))
 (segment (start 116.34 88.596396) (end 127.528604 99.785) (width 0.25) (layer "B.Cu") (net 17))
 (segment (start 118.14 86.871396) (end 117.49 87.521396) (width 0.25) (layer "B.Cu") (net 17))
 (segment (start 117.49 87.96) (end 117.49 88.46) (width 0.25) (layer "B.Cu") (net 17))
 (segment (start 129.54 88.9) (end 130.5 88.9) (width 0.25) (layer "B.Cu") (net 17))
 (segment (start 116.84 86.36) (end 116.84 83.82) (width 0.25) (layer "B.Cu") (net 17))
 (segment (start 117.565 88.535) (end 119.165 88.535) (width 0.25) (layer "B.Cu") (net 17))
 (segment (start 119.38 81.28) (end 124.46 81.28) (width 0.25) (layer "B.Cu") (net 17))
 (segment (start 127.528604 99.785) (end 129.840305 99.785) (width 0.25) (layer "B.Cu") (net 17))
 (segment (start 144.78 89.93) (end 144.78 90.7755) (width 0.25) (layer "B.Cu") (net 17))
 (segment (start 116.34 86.86) (end 116.34 88.596396) (width 0.25) (layer "B.Cu") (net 17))
 (segment (start 118.14 85.06) (end 120.59 82.61) (width 0.25) (layer "B.Cu") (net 17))
 (segment (start 129.840305 99.785) (end 130.265 99.360305) (width 0.25) (layer "B.Cu") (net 17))
 (segment (start 117.49 87.521396) (end 117.49 87.96) (width 0.25) (layer "B.Cu") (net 17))
 (segment (start 144.78 90.7755) (end 142.935451 92.620049) (width 0.25) (layer "B.Cu") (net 17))
 (segment (start 142.935451 92.620049) (end 143.169951 92.620049) (width 0.25) (layer "B.Cu") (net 17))
 (segment (start 119.29 88.41) (end 129.05 88.41) (width 0.25) (layer "B.Cu") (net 17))
 (segment (start 124.46 81.28) (end 125.79 82.61) (width 0.25) (layer "B.Cu") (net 17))
 (segment (start 117.49 88.46) (end 117.565 88.535) (width 0.25) (layer "B.Cu") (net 17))
 (segment (start 116.84 83.82) (end 119.38 81.28) (width 0.25) (layer "B.Cu") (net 17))
 (segment (start 116.84 86.36) (end 116.34 86.86) (width 0.25) (layer "B.Cu") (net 17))
 (segment (start 120.59 82.61) (end 121.92 82.61) (width 0.25) (layer "B.Cu") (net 17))
 (segment (start 130.265 89.625) (end 129.54 88.9) (width 0.25) (layer "B.Cu") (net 17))
 (segment (start 118.14 86.36) (end 118.14 85.06) (width 0.25) (layer "B.Cu") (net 17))
 (segment (start 130.265 99.360305) (end 130.265 89.625) (width 0.25) (layer "B.Cu") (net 17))
 (segment (start 119.165 88.535) (end 119.29 88.41) (width 0.25) (layer "B.Cu") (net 17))
 (segment (start 182.88 82.5925) (end 182.88 76.2) (width 0.25) (layer "F.Cu") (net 15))
 (segment (start 182.88 76.2) (end 180.34 73.66) (width 0.25) (layer "F.Cu") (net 15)))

